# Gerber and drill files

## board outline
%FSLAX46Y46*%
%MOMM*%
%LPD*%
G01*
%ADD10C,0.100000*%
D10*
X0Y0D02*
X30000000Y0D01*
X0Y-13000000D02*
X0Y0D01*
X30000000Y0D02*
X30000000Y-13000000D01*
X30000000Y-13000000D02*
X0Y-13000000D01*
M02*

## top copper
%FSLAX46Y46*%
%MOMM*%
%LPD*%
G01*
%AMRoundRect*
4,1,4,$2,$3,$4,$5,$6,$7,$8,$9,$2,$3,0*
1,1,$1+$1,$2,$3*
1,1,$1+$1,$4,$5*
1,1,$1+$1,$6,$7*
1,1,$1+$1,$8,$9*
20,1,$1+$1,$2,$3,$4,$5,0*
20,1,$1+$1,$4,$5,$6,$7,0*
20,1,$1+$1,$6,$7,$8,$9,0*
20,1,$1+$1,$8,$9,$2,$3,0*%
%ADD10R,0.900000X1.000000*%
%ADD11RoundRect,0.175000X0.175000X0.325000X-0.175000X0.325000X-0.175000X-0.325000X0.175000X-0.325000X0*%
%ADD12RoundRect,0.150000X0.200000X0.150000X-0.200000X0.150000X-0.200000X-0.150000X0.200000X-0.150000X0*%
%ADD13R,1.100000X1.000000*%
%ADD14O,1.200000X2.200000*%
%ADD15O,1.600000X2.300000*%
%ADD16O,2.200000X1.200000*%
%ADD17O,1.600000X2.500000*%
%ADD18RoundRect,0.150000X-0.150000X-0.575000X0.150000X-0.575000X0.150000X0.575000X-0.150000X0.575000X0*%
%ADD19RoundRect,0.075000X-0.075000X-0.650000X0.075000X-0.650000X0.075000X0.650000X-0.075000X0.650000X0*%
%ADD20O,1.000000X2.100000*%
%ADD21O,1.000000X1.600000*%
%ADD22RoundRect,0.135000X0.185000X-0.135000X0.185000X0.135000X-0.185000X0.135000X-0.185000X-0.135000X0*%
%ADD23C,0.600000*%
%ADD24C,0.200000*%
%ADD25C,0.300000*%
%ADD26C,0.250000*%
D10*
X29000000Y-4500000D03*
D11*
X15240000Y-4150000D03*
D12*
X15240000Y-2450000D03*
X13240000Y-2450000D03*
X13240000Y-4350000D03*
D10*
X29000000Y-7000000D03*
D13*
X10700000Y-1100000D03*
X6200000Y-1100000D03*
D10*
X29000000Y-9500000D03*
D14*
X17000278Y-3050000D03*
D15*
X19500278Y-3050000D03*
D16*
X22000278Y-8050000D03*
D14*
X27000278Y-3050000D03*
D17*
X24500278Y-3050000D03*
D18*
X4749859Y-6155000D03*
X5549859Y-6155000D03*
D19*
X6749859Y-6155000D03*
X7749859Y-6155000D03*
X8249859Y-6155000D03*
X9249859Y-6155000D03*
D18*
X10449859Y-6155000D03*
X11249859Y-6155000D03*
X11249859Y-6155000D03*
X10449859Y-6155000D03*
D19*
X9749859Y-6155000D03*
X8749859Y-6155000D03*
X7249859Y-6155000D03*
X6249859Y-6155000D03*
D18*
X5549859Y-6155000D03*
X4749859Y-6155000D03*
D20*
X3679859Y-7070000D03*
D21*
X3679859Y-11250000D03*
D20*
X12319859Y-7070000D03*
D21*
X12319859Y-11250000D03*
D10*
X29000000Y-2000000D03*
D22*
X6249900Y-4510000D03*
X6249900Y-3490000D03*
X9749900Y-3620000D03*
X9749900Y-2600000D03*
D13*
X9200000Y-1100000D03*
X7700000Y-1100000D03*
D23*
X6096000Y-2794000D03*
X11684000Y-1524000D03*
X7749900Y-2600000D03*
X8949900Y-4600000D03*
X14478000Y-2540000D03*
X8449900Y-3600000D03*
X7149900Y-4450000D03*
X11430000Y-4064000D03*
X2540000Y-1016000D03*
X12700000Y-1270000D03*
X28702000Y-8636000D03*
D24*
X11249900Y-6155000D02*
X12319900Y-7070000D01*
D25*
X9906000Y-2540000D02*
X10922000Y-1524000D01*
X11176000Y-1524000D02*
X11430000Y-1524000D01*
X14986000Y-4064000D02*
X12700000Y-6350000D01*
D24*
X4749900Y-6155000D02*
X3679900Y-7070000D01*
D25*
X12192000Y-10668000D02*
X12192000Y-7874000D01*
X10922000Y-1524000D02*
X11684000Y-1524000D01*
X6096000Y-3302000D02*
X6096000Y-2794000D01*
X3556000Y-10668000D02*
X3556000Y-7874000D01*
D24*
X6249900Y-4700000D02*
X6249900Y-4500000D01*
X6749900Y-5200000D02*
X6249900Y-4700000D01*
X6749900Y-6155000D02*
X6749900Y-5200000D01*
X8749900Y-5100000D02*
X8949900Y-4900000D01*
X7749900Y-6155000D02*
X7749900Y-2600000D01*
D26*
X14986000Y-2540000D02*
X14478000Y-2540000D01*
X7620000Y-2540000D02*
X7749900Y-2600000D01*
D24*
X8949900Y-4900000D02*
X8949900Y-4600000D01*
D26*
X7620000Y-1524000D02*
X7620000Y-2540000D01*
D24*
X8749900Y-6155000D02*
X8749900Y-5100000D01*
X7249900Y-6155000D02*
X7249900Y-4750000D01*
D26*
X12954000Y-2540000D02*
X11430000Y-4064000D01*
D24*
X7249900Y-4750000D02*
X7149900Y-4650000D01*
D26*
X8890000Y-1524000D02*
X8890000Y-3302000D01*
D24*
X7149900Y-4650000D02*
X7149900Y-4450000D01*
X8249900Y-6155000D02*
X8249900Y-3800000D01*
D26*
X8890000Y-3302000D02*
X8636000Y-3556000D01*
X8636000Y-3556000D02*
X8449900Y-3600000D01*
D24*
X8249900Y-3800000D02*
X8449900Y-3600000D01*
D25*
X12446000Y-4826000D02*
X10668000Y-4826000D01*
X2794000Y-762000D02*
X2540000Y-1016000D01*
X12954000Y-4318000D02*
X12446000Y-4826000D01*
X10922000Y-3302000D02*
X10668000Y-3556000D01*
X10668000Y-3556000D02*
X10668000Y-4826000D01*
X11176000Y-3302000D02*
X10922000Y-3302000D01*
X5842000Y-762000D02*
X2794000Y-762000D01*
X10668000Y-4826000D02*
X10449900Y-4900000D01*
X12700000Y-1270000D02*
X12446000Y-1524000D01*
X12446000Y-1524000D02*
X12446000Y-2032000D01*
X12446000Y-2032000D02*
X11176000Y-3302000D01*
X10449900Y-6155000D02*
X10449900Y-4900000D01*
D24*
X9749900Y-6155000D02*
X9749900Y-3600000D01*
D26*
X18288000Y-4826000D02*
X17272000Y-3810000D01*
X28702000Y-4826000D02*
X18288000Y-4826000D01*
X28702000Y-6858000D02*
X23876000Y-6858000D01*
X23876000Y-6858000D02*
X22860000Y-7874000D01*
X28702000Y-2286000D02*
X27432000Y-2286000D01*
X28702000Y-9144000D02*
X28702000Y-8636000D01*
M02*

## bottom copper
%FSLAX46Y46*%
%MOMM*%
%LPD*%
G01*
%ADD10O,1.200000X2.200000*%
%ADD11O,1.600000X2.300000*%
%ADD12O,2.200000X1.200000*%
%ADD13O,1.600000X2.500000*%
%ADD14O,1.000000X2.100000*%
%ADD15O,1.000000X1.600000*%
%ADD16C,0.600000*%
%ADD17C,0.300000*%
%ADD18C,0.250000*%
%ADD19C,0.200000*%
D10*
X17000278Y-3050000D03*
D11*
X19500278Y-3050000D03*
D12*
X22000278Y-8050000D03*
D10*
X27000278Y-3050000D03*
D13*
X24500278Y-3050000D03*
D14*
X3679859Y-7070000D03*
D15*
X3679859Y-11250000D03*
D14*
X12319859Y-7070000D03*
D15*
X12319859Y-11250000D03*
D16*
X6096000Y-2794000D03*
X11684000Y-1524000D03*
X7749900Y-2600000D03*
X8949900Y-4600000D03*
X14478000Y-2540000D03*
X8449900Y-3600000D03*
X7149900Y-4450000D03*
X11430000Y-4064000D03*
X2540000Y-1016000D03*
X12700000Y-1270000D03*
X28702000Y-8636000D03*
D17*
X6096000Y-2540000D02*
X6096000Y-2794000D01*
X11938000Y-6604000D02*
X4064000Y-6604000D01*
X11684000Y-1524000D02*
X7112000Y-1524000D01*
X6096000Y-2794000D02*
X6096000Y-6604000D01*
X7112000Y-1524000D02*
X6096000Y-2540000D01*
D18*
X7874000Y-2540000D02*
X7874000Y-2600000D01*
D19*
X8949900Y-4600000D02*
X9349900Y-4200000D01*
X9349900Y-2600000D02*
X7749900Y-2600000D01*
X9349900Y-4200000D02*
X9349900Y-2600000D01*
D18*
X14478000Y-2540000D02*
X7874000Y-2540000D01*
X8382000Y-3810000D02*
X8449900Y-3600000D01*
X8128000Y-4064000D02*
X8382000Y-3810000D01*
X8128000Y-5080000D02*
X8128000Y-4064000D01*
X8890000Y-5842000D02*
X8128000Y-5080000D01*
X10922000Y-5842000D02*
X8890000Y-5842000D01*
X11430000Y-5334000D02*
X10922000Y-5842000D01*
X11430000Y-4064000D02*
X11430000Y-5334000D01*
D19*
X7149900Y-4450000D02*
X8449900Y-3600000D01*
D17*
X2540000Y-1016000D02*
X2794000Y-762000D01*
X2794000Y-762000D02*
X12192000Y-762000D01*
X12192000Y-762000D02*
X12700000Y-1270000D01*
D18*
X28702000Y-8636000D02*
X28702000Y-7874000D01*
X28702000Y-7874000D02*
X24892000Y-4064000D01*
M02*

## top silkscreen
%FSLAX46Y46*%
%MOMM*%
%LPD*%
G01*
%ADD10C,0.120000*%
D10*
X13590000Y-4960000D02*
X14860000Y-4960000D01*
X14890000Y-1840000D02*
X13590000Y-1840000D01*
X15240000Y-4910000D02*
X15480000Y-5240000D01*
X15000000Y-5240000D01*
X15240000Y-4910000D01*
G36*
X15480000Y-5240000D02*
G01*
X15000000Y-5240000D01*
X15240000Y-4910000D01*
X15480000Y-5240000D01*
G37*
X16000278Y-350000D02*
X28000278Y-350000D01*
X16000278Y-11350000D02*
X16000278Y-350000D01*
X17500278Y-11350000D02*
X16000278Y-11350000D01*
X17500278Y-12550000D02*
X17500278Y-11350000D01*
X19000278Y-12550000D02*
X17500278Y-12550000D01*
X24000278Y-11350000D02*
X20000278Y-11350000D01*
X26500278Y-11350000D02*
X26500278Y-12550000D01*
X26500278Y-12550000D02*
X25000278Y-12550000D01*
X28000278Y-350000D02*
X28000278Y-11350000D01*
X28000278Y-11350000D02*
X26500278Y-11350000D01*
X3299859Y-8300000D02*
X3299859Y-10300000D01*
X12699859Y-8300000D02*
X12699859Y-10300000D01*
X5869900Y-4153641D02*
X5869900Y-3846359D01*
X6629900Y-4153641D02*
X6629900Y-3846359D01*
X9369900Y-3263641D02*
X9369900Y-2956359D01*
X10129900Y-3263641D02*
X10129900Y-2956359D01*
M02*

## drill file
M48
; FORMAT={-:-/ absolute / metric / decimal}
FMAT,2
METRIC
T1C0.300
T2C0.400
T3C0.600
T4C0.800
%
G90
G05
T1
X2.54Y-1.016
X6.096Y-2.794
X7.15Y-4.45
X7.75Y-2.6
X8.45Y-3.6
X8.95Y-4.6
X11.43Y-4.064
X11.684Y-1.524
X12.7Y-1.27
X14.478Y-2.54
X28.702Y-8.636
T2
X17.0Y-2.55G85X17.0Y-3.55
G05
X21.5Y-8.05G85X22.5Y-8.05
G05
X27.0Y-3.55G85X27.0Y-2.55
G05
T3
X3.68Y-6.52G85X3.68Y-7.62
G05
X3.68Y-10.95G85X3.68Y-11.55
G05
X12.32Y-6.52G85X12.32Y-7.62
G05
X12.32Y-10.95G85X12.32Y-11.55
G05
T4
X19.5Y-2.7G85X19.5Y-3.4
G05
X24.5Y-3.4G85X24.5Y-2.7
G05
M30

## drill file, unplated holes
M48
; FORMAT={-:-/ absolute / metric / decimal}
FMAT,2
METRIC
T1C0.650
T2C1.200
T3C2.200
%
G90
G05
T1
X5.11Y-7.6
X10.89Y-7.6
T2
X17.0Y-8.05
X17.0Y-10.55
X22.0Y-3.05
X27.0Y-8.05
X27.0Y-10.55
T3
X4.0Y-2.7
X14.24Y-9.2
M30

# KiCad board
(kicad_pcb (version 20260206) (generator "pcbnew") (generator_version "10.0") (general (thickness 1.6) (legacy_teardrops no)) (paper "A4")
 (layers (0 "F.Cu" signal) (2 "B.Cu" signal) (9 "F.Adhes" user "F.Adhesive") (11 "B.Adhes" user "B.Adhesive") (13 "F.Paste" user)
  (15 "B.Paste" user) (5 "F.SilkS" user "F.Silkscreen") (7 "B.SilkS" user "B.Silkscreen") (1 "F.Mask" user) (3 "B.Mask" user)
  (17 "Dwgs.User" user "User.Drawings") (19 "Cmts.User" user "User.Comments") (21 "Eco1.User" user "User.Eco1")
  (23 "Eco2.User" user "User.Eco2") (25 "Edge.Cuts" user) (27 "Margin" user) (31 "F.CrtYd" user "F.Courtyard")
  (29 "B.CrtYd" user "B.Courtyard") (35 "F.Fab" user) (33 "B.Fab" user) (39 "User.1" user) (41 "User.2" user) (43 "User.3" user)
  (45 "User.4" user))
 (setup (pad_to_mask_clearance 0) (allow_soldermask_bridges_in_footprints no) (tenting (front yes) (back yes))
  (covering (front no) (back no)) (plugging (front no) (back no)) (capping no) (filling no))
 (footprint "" (layer "F.Cu") (at 29 4.5)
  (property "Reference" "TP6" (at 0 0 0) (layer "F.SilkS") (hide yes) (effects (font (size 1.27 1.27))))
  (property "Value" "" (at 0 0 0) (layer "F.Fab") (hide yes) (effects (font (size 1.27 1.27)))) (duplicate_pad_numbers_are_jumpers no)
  (pad "1" smd rect (at 0 0) (size 0.9 1) (layers "F.Cu" "F.Mask" "F.Paste") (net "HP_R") (thermal_bridge_angle 45)))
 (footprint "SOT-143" (layer "F.Cu") (at 14.24 3.4 180)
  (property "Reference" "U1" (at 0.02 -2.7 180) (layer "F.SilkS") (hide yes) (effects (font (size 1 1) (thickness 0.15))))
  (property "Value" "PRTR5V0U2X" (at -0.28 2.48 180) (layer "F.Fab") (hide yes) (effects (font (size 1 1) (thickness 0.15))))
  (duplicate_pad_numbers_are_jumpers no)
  (fp_line (start 0.65 -1.56) (end -0.62 -1.56) (stroke (width 0.12) (type solid)) (layer "F.SilkS"))
  (fp_line (start -0.65 1.56) (end 0.65 1.56) (stroke (width 0.12) (type solid)) (layer "F.SilkS"))
  (fp_poly
   (pts (xy -1 -1.51) (xy -1.24 -1.84) (xy -0.76 -1.84) (xy -1 -1.51)) (stroke (width 0.12) (type solid)) (fill yes) (layer "F.SilkS"))
  (pad "1" smd roundrect (at -1 -0.75 180) (size 0.7 1) (layers "F.Cu" "F.Mask" "F.Paste") (roundrect_rratio 0.25) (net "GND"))
  (pad "2" smd roundrect (at -1 0.95 180) (size 0.7 0.6) (layers "F.Cu" "F.Mask" "F.Paste") (roundrect_rratio 0.25) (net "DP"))
  (pad "3" smd roundrect (at 1 0.95 180) (size 0.7 0.6) (layers "F.Cu" "F.Mask" "F.Paste") (roundrect_rratio 0.25) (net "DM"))
  (pad "4" smd roundrect (at 1 -0.95 180) (size 0.7 0.6) (layers "F.Cu" "F.Mask" "F.Paste") (roundrect_rratio 0.25) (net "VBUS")))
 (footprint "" (layer "F.Cu") (at 29 7)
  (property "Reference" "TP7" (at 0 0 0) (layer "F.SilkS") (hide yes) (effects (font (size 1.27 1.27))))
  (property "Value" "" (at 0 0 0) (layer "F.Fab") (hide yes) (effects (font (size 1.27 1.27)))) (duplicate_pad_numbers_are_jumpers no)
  (pad "1" smd rect (at 0 0) (size 0.9 1) (layers "F.Cu" "F.Mask" "F.Paste") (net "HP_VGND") (thermal_bridge_angle 45)))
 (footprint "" (layer "F.Cu") (at 10.7 1.1)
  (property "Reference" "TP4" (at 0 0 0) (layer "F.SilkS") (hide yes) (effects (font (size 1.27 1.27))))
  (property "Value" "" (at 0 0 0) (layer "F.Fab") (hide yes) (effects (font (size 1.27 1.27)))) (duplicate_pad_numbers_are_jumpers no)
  (pad "1" smd rect (at 0 0) (size 1.1 1) (layers "F.Cu" "F.Mask" "F.Paste") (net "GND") (thermal_bridge_angle 45)))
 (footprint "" (layer "F.Cu") (at 6.2 1.1)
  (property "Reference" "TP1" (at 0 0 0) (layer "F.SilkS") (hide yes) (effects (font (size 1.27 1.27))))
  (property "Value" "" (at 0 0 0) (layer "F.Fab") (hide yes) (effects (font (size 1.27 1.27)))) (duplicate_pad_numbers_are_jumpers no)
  (pad "1" smd rect (at 0 0) (size 1.1 1) (layers "F.Cu" "F.Mask" "F.Paste") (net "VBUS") (thermal_bridge_angle 45)))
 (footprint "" (layer "F.Cu") (at 29 9.5)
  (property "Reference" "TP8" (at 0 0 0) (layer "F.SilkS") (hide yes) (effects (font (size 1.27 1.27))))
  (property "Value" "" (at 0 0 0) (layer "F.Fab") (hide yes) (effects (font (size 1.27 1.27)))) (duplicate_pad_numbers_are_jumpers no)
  (pad "1" smd rect (at 0 0) (size 0.9 1) (layers "F.Cu" "F.Mask" "F.Paste") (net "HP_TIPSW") (thermal_bridge_angle 45)))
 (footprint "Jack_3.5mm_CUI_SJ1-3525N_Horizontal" (layer "F.Cu") (at 22.000278 8.05)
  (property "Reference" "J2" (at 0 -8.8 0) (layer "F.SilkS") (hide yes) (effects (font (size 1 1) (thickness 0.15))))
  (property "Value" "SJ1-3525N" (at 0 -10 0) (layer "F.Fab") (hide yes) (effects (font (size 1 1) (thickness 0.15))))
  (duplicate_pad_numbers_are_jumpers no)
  (fp_line (start -6 -7.7) (end 6 -7.7) (stroke (width 0.12) (type solid)) (layer "F.SilkS"))
  (fp_line (start -6 3.3) (end -6 -7.7) (stroke (width 0.12) (type solid)) (layer "F.SilkS"))
  (fp_line (start -4.5 3.3) (end -6 3.3) (stroke (width 0.12) (type solid)) (layer "F.SilkS"))
  (fp_line (start -4.5 4.5) (end -4.5 3.3) (stroke (width 0.12) (type solid)) (layer "F.SilkS"))
  (fp_line (start -3 4.5) (end -4.5 4.5) (stroke (width 0.12) (type solid)) (layer "F.SilkS"))
  (fp_line (start 2 3.3) (end -2 3.3) (stroke (width 0.12) (type solid)) (layer "F.SilkS"))
  (fp_line (start 4.5 3.3) (end 4.5 4.5) (stroke (width 0.12) (type solid)) (layer "F.SilkS"))
  (fp_line (start 4.5 4.5) (end 3 4.5) (stroke (width 0.12) (type solid)) (layer "F.SilkS"))
  (fp_line (start 6 -7.7) (end 6 3.3) (stroke (width 0.12) (type solid)) (layer "F.SilkS"))
  (fp_line (start 6 3.3) (end 4.5 3.3) (stroke (width 0.12) (type solid)) (layer "F.SilkS"))
  (pad "" np_thru_hole circle (at -5 0) (size 1.2 1.2) (drill 1.2) (layers "*.Cu" "*.Mask"))
  (pad "" np_thru_hole circle (at -5 2.5) (size 1.2 1.2) (drill 1.2) (layers "*.Cu" "*.Mask"))
  (pad "" np_thru_hole circle (at 0 -5) (size 1.2 1.2) (drill 1.2) (layers "*.Cu" "*.Mask"))
  (pad "" np_thru_hole circle (at 5 0) (size 1.2 1.2) (drill 1.2) (layers "*.Cu" "*.Mask"))
  (pad "" np_thru_hole circle (at 5 2.5) (size 1.2 1.2) (drill 1.2) (layers "*.Cu" "*.Mask"))
  (pad "R" thru_hole oval (at -5 -5) (size 1.2 2.2) (drill oval 0.4 1.4) (layers "*.Cu" "*.Mask") (remove_unused_layers no) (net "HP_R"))
  (pad "RN" thru_hole oval (at -2.5 -5) (size 1.6 2.3) (drill oval 0.8 1.5) (layers "*.Cu" "*.Mask") (remove_unused_layers no))
  (pad "S" thru_hole oval (at 0 0) (size 2.2 1.2) (drill oval 1.4 0.4) (layers "*.Cu" "*.Mask") (remove_unused_layers no) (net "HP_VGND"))
  (pad "T" thru_hole oval (at 5 -5 180) (size 1.2 2.2) (drill oval 0.4 1.4) (layers "*.Cu" "*.Mask") (remove_unused_layers no) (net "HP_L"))
  (pad "TN" thru_hole oval (at 2.5 -5 180) (size 1.6 2.5) (drill oval 0.8 1.5) (layers "*.Cu" "*.Mask") (remove_unused_layers no)
   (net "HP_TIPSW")))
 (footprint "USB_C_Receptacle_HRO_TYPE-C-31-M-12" (layer "F.Cu") (at 7.999859 10.2)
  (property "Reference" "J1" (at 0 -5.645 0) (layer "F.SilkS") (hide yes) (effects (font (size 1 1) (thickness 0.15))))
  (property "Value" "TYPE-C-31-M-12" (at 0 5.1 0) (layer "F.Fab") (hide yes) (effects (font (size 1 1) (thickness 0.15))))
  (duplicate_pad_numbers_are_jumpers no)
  (fp_line (start -4.7 -1.9) (end -4.7 0.1) (stroke (width 0.12) (type solid)) (layer "F.SilkS"))
  (fp_line (start 4.7 -1.9) (end 4.7 0.1) (stroke (width 0.12) (type solid)) (layer "F.SilkS"))
  (pad "" np_thru_hole circle (at -2.89 -2.6) (size 0.65 0.65) (drill 0.65) (layers "*.Cu" "*.Mask"))
  (pad "" np_thru_hole circle (at 2.89 -2.6) (size 0.65 0.65) (drill 0.65) (layers "*.Cu" "*.Mask"))
  (pad "A1" smd roundrect (at -3.25 -4.045) (size 0.6 1.45) (layers "F.Cu" "F.Mask" "F.Paste") (roundrect_rratio 0.25) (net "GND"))
  (pad "A4" smd roundrect (at -2.45 -4.045) (size 0.6 1.45) (layers "F.Cu" "F.Mask" "F.Paste") (roundrect_rratio 0.25) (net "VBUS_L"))
  (pad "A5" smd roundrect (at -1.25 -4.045) (size 0.3 1.45) (layers "F.Cu" "F.Mask" "F.Paste") (roundrect_rratio 0.25) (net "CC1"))
  (pad "A6" smd roundrect (at -0.25 -4.045) (size 0.3 1.45) (layers "F.Cu" "F.Mask" "F.Paste") (roundrect_rratio 0.25) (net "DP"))
  (pad "A7" smd roundrect (at 0.25 -4.045) (size 0.3 1.45) (layers "F.Cu" "F.Mask" "F.Paste") (roundrect_rratio 0.25) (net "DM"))
  (pad "A8" smd roundrect (at 1.25 -4.045) (size 0.3 1.45) (layers "F.Cu" "F.Mask" "F.Paste") (roundrect_rratio 0.25))
  (pad "A9" smd roundrect (at 2.45 -4.045) (size 0.6 1.45) (layers "F.Cu" "F.Mask" "F.Paste") (roundrect_rratio 0.25) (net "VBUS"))
  (pad "A12" smd roundrect (at 3.25 -4.045) (size 0.6 1.45) (layers "F.Cu" "F.Mask" "F.Paste") (roundrect_rratio 0.25) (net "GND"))
  (pad "B1" smd roundrect (at 3.25 -4.045) (size 0.6 1.45) (layers "F.Cu" "F.Mask" "F.Paste") (roundrect_rratio 0.25) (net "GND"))
  (pad "B4" smd roundrect (at 2.45 -4.045) (size 0.6 1.45) (layers "F.Cu" "F.Mask" "F.Paste") (roundrect_rratio 0.25) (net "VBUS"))
  (pad "B5" smd roundrect (at 1.75 -4.045) (size 0.3 1.45) (layers "F.Cu" "F.Mask" "F.Paste") (roundrect_rratio 0.25) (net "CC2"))
  (pad "B6" smd roundrect (at 0.75 -4.045) (size 0.3 1.45) (layers "F.Cu" "F.Mask" "F.Paste") (roundrect_rratio 0.25) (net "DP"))
  (pad "B7" smd roundrect (at -0.75 -4.045) (size 0.3 1.45) (layers "F.Cu" "F.Mask" "F.Paste") (roundrect_rratio 0.25) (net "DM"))
  (pad "B8" smd roundrect (at -1.75 -4.045) (size 0.3 1.45) (layers "F.Cu" "F.Mask" "F.Paste") (roundrect_rratio 0.25))
  (pad "B9" smd roundrect (at -2.45 -4.045) (size 0.6 1.45) (layers "F.Cu" "F.Mask" "F.Paste") (roundrect_rratio 0.25) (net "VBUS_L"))
  (pad "B12" smd roundrect (at -3.25 -4.045) (size 0.6 1.45) (layers "F.Cu" "F.Mask" "F.Paste") (roundrect_rratio 0.25) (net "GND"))
  (pad "SH" thru_hole oval (at -4.32 -3.13) (size 1 2.1) (drill oval 0.6 1.7) (layers "*.Cu" "*.Mask") (remove_unused_layers no) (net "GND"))
  (pad "SH" thru_hole oval (at -4.32 1.05) (size 1 1.6) (drill oval 0.6 1.2) (layers "*.Cu" "*.Mask") (remove_unused_layers no) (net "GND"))
  (pad "SH" thru_hole oval (at 4.32 -3.13) (size 1 2.1) (drill oval 0.6 1.7) (layers "*.Cu" "*.Mask") (remove_unused_layers no) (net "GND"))
  (pad "SH" thru_hole oval (at 4.32 1.05) (size 1 1.6) (drill oval 0.6 1.2) (layers "*.Cu" "*.Mask") (remove_unused_layers no) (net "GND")))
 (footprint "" (layer "F.Cu") (at 29 2)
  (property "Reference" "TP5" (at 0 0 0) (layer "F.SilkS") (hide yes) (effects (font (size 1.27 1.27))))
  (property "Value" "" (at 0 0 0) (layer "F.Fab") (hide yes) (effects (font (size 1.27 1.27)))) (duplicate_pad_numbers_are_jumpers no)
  (pad "1" smd rect (at 0 0) (size 0.9 1) (layers "F.Cu" "F.Mask" "F.Paste") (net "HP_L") (thermal_bridge_angle 45)))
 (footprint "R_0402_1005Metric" (layer "F.Cu") (at 6.2499 4 90)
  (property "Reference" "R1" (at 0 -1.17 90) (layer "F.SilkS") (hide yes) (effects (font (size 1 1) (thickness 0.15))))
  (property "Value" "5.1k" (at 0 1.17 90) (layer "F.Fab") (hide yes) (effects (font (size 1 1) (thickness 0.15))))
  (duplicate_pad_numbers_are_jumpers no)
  (fp_line (start -0.153641 -0.38) (end 0.153641 -0.38) (stroke (width 0.12) (type solid)) (layer "F.SilkS"))
  (fp_line (start -0.153641 0.38) (end 0.153641 0.38) (stroke (width 0.12) (type solid)) (layer "F.SilkS"))
  (pad "1" smd roundrect (at -0.51 0 90) (size 0.54 0.64) (layers "F.Cu" "F.Mask" "F.Paste") (roundrect_rratio 0.25) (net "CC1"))
  (pad "2" smd roundrect (at 0.51 0 90) (size 0.54 0.64) (layers "F.Cu" "F.Mask" "F.Paste") (roundrect_rratio 0.25) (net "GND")))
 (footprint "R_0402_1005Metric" (layer "F.Cu") (at 9.7499 3.11 90)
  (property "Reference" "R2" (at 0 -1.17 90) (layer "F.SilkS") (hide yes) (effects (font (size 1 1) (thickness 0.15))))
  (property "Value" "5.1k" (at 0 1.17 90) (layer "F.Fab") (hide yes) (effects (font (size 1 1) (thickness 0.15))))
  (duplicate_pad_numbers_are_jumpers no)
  (fp_line (start -0.153641 -0.38) (end 0.153641 -0.38) (stroke (width 0.12) (type solid)) (layer "F.SilkS"))
  (fp_line (start -0.153641 0.38) (end 0.153641 0.38) (stroke (width 0.12) (type solid)) (layer "F.SilkS"))
  (pad "1" smd roundrect (at -0.51 0 90) (size 0.54 0.64) (layers "F.Cu" "F.Mask" "F.Paste") (roundrect_rratio 0.25) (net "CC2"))
  (pad "2" smd roundrect (at 0.51 0 90) (size 0.54 0.64) (layers "F.Cu" "F.Mask" "F.Paste") (roundrect_rratio 0.25) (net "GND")))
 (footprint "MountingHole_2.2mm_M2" (layer "F.Cu") (at 14.24 9.2)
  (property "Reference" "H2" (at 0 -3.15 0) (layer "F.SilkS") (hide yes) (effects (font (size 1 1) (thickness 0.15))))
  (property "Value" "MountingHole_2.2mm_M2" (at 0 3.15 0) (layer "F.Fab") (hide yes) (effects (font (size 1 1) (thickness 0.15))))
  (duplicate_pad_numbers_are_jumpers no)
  (pad "" np_thru_hole circle (at 0 0) (size 2.2 2.2) (drill 2.2) (layers "*.Cu" "*.Mask")))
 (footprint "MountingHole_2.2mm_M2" (layer "F.Cu") (at 4 2.699999)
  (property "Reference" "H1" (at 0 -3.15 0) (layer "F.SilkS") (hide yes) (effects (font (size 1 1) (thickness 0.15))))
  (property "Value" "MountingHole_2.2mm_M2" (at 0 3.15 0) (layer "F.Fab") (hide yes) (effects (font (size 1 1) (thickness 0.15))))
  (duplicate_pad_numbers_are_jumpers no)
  (pad "" np_thru_hole circle (at 0 0) (size 2.2 2.2) (drill 2.2) (layers "*.Cu" "*.Mask")))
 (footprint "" (layer "F.Cu") (at 9.2 1.1)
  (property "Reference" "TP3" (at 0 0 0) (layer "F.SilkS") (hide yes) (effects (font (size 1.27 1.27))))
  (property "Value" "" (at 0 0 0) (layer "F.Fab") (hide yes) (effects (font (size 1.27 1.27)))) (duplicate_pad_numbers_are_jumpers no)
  (pad "1" smd rect (at 0 0) (size 1.1 1) (layers "F.Cu" "F.Mask" "F.Paste") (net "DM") (thermal_bridge_angle 45)))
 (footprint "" (layer "F.Cu") (at 7.7 1.1)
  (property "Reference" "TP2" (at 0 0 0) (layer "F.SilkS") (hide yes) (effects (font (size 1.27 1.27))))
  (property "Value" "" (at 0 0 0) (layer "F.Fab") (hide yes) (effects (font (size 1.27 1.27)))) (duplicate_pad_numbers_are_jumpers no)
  (pad "1" smd rect (at 0 0) (size 1.1 1) (layers "F.Cu" "F.Mask" "F.Paste") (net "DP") (thermal_bridge_angle 45)))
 (gr_line (start 0 0) (end 30 0) (stroke (width 0.1) (type default)) (layer "Edge.Cuts"))
 (gr_line (start 0 13) (end 0 0) (stroke (width 0.1) (type default)) (layer "Edge.Cuts"))
 (gr_line (start 30 0) (end 30 13) (stroke (width 0.1) (type default)) (layer "Edge.Cuts"))
 (gr_line (start 30 13) (end 0 13) (stroke (width 0.1) (type default)) (layer "Edge.Cuts"))
 (segment (start 11.2499 6.155) (end 12.3199 7.07) (width 0.2) (layer "F.Cu") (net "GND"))
 (segment (start 9.906 2.54) (end 10.922 1.524) (width 0.3) (layer "F.Cu") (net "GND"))
 (segment (start 11.176 1.524) (end 11.43 1.524) (width 0.3) (layer "F.Cu") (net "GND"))
 (segment (start 14.986 4.064) (end 12.7 6.35) (width 0.3) (layer "F.Cu") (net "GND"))
 (segment (start 4.7499 6.155) (end 3.6799 7.07) (width 0.2) (layer "F.Cu") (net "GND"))
 (segment (start 12.192 10.668) (end 12.192 7.874) (width 0.3) (layer "F.Cu") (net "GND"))
 (segment (start 10.922 1.524) (end 11.684 1.524) (width 0.3) (layer "F.Cu") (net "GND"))
 (segment (start 6.096 3.302) (end 6.096 2.794) (width 0.3) (layer "F.Cu") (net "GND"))
 (segment (start 3.556 10.668) (end 3.556 7.874) (width 0.3) (layer "F.Cu") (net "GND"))
 (via (at 6.096 2.794) (size 0.6) (drill 0.3) (layers "F.Cu" "B.Cu") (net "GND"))
 (via (at 11.684 1.524) (size 0.6) (drill 0.3) (layers "F.Cu" "B.Cu") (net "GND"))
 (segment (start 6.096 2.54) (end 6.096 2.794) (width 0.3) (layer "B.Cu") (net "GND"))
 (segment (start 11.938 6.604) (end 4.064 6.604) (width 0.3) (layer "B.Cu") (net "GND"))
 (segment (start 11.684 1.524) (end 7.112 1.524) (width 0.3) (layer "B.Cu") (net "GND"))
 (segment (start 6.096 2.794) (end 6.096 6.604) (width 0.3) (layer "B.Cu") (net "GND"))
 (segment (start 7.112 1.524) (end 6.096 2.54) (width 0.3) (layer "B.Cu") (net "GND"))
 (segment (start 6.2499 4.7) (end 6.2499 4.5) (width 0.2) (layer "F.Cu") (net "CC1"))
 (segment (start 6.7499 5.2) (end 6.2499 4.7) (width 0.2) (layer "F.Cu") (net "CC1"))
 (segment (start 6.7499 6.155) (end 6.7499 5.2) (width 0.2) (layer "F.Cu") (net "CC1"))
 (segment (start 8.7499 5.1) (end 8.9499 4.9) (width 0.2) (layer "F.Cu") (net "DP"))
 (segment (start 7.7499 6.155) (end 7.7499 2.6) (width 0.2) (layer "F.Cu") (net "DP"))
 (segment (start 14.986 2.54) (end 14.478 2.54) (width 0.25) (layer "F.Cu") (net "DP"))
 (segment (start 7.62 2.54) (end 7.7499 2.6) (width 0.25) (layer "F.Cu") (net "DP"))
 (segment (start 8.9499 4.9) (end 8.9499 4.6) (width 0.2) (layer "F.Cu") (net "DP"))
 (segment (start 7.62 1.524) (end 7.62 2.54) (width 0.25) (layer "F.Cu") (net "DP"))
 (segment (start 8.7499 6.155) (end 8.7499 5.1) (width 0.2) (layer "F.Cu") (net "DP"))
 (via (at 7.7499 2.6) (size 0.6) (drill 0.3) (layers "F.Cu" "B.Cu") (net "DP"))
 (via (at 8.9499 4.6) (size 0.6) (drill 0.3) (layers "F.Cu" "B.Cu") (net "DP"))
 (via (at 14.478 2.54) (size 0.6) (drill 0.3) (layers "F.Cu" "B.Cu") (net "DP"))
 (segment (start 7.874 2.54) (end 7.874 2.6) (width 0.25) (layer "B.Cu") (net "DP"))
 (segment (start 8.9499 4.6) (end 9.3499 4.2) (width 0.2) (layer "B.Cu") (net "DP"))
 (segment (start 9.3499 2.6) (end 7.7499 2.6) (width 0.2) (layer "B.Cu") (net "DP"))
 (segment (start 9.3499 4.2) (end 9.3499 2.6) (width 0.2) (layer "B.Cu") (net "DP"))
 (segment (start 14.478 2.54) (end 7.874 2.54) (width 0.25) (layer "B.Cu") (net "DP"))
 (segment (start 7.2499 6.155) (end 7.2499 4.75) (width 0.2) (layer "F.Cu") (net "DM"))
 (segment (start 12.954 2.54) (end 11.43 4.064) (width 0.25) (layer "F.Cu") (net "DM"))
 (segment (start 7.2499 4.75) (end 7.1499 4.65) (width 0.2) (layer "F.Cu") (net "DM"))
 (segment (start 8.89 1.524) (end 8.89 3.302) (width 0.25) (layer "F.Cu") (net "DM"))
 (segment (start 7.1499 4.65) (end 7.1499 4.45) (width 0.2) (layer "F.Cu") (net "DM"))
 (segment (start 8.2499 6.155) (end 8.2499 3.8) (width 0.2) (layer "F.Cu") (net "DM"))
 (segment (start 8.89 3.302) (end 8.636 3.556) (width 0.25) (layer "F.Cu") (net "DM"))
 (segment (start 8.636 3.556) (end 8.4499 3.6) (width 0.25) (layer "F.Cu") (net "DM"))
 (segment (start 8.2499 3.8) (end 8.4499 3.6) (width 0.2) (layer "F.Cu") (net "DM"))
 (via (at 8.4499 3.6) (size 0.6) (drill 0.3) (layers "F.Cu" "B.Cu") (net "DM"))
 (via (at 7.1499 4.45) (size 0.6) (drill 0.3) (layers "F.Cu" "B.Cu") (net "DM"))
 (via (at 11.43 4.064) (size 0.6) (drill 0.3) (layers "F.Cu" "B.Cu") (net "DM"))
 (segment (start 8.382 3.81) (end 8.4499 3.6) (width 0.25) (layer "B.Cu") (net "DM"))
 (segment (start 8.128 4.064) (end 8.382 3.81) (width 0.25) (layer "B.Cu") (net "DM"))
 (segment (start 8.128 5.08) (end 8.128 4.064) (width 0.25) (layer "B.Cu") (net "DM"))
 (segment (start 8.89 5.842) (end 8.128 5.08) (width 0.25) (layer "B.Cu") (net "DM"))
 (segment (start 10.922 5.842) (end 8.89 5.842) (width 0.25) (layer "B.Cu") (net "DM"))
 (segment (start 11.43 5.334) (end 10.922 5.842) (width 0.25) (layer "B.Cu") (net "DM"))
 (segment (start 11.43 4.064) (end 11.43 5.334) (width 0.25) (layer "B.Cu") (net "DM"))
 (segment (start 7.1499 4.45) (end 8.4499 3.6) (width 0.2) (layer "B.Cu") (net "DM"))
 (segment (start 12.446 4.826) (end 10.668 4.826) (width 0.3) (layer "F.Cu") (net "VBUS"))
 (segment (start 2.794 0.762) (end 2.54 1.016) (width 0.3) (layer "F.Cu") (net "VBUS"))
 (segment (start 12.954 4.318) (end 12.446 4.826) (width 0.3) (layer "F.Cu") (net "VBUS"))
 (segment (start 10.922 3.302) (end 10.668 3.556) (width 0.3) (layer "F.Cu") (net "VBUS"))
 (segment (start 10.668 3.556) (end 10.668 4.826) (width 0.3) (layer "F.Cu") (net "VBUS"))
 (segment (start 11.176 3.302) (end 10.922 3.302) (width 0.3) (layer "F.Cu") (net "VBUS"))
 (segment (start 5.842 0.762) (end 2.794 0.762) (width 0.3) (layer "F.Cu") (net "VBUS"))
 (segment (start 10.668 4.826) (end 10.4499 4.9) (width 0.3) (layer "F.Cu") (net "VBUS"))
 (segment (start 12.7 1.27) (end 12.446 1.524) (width 0.3) (layer "F.Cu") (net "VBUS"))
 (segment (start 12.446 1.524) (end 12.446 2.032) (width 0.3) (layer "F.Cu") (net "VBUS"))
 (segment (start 12.446 2.032) (end 11.176 3.302) (width 0.3) (layer "F.Cu") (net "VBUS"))
 (segment (start 10.4499 6.155) (end 10.4499 4.9) (width 0.3) (layer "F.Cu") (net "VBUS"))
 (via (at 2.54 1.016) (size 0.6) (drill 0.3) (layers "F.Cu" "B.Cu") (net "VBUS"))
 (via (at 12.7 1.27) (size 0.6) (drill 0.3) (layers "F.Cu" "B.Cu") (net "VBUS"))
 (segment (start 2.54 1.016) (end 2.794 0.762) (width 0.3) (layer "B.Cu") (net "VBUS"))
 (segment (start 2.794 0.762) (end 12.192 0.762) (width 0.3) (layer "B.Cu") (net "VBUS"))
 (segment (start 12.192 0.762) (end 12.7 1.27) (width 0.3) (layer "B.Cu") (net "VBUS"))
 (segment (start 9.7499 6.155) (end 9.7499 3.6) (width 0.2) (layer "F.Cu") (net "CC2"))
 (segment (start 18.288 4.826) (end 17.272 3.81) (width 0.25) (layer "F.Cu") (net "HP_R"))
 (segment (start 28.702 4.826) (end 18.288 4.826) (width 0.25) (layer "F.Cu") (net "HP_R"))
 (segment (start 28.702 6.858) (end 23.876 6.858) (width 0.25) (layer "F.Cu") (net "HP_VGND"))
 (segment (start 23.876 6.858) (end 22.86 7.874) (width 0.25) (layer "F.Cu") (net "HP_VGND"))
 (segment (start 28.702 2.286) (end 27.432 2.286) (width 0.25) (layer "F.Cu") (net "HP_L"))
 (segment (start 28.702 9.144) (end 28.702 8.636) (width 0.25) (layer "F.Cu") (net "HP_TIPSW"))
 (via (at 28.702 8.636) (size 0.6) (drill 0.3) (layers "F.Cu" "B.Cu") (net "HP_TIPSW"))
 (segment (start 28.702 8.636) (end 28.702 7.874) (width 0.25) (layer "B.Cu") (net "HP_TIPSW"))
 (segment (start 28.702 7.874) (end 24.892 4.064) (width 0.25) (layer "B.Cu") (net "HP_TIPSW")))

